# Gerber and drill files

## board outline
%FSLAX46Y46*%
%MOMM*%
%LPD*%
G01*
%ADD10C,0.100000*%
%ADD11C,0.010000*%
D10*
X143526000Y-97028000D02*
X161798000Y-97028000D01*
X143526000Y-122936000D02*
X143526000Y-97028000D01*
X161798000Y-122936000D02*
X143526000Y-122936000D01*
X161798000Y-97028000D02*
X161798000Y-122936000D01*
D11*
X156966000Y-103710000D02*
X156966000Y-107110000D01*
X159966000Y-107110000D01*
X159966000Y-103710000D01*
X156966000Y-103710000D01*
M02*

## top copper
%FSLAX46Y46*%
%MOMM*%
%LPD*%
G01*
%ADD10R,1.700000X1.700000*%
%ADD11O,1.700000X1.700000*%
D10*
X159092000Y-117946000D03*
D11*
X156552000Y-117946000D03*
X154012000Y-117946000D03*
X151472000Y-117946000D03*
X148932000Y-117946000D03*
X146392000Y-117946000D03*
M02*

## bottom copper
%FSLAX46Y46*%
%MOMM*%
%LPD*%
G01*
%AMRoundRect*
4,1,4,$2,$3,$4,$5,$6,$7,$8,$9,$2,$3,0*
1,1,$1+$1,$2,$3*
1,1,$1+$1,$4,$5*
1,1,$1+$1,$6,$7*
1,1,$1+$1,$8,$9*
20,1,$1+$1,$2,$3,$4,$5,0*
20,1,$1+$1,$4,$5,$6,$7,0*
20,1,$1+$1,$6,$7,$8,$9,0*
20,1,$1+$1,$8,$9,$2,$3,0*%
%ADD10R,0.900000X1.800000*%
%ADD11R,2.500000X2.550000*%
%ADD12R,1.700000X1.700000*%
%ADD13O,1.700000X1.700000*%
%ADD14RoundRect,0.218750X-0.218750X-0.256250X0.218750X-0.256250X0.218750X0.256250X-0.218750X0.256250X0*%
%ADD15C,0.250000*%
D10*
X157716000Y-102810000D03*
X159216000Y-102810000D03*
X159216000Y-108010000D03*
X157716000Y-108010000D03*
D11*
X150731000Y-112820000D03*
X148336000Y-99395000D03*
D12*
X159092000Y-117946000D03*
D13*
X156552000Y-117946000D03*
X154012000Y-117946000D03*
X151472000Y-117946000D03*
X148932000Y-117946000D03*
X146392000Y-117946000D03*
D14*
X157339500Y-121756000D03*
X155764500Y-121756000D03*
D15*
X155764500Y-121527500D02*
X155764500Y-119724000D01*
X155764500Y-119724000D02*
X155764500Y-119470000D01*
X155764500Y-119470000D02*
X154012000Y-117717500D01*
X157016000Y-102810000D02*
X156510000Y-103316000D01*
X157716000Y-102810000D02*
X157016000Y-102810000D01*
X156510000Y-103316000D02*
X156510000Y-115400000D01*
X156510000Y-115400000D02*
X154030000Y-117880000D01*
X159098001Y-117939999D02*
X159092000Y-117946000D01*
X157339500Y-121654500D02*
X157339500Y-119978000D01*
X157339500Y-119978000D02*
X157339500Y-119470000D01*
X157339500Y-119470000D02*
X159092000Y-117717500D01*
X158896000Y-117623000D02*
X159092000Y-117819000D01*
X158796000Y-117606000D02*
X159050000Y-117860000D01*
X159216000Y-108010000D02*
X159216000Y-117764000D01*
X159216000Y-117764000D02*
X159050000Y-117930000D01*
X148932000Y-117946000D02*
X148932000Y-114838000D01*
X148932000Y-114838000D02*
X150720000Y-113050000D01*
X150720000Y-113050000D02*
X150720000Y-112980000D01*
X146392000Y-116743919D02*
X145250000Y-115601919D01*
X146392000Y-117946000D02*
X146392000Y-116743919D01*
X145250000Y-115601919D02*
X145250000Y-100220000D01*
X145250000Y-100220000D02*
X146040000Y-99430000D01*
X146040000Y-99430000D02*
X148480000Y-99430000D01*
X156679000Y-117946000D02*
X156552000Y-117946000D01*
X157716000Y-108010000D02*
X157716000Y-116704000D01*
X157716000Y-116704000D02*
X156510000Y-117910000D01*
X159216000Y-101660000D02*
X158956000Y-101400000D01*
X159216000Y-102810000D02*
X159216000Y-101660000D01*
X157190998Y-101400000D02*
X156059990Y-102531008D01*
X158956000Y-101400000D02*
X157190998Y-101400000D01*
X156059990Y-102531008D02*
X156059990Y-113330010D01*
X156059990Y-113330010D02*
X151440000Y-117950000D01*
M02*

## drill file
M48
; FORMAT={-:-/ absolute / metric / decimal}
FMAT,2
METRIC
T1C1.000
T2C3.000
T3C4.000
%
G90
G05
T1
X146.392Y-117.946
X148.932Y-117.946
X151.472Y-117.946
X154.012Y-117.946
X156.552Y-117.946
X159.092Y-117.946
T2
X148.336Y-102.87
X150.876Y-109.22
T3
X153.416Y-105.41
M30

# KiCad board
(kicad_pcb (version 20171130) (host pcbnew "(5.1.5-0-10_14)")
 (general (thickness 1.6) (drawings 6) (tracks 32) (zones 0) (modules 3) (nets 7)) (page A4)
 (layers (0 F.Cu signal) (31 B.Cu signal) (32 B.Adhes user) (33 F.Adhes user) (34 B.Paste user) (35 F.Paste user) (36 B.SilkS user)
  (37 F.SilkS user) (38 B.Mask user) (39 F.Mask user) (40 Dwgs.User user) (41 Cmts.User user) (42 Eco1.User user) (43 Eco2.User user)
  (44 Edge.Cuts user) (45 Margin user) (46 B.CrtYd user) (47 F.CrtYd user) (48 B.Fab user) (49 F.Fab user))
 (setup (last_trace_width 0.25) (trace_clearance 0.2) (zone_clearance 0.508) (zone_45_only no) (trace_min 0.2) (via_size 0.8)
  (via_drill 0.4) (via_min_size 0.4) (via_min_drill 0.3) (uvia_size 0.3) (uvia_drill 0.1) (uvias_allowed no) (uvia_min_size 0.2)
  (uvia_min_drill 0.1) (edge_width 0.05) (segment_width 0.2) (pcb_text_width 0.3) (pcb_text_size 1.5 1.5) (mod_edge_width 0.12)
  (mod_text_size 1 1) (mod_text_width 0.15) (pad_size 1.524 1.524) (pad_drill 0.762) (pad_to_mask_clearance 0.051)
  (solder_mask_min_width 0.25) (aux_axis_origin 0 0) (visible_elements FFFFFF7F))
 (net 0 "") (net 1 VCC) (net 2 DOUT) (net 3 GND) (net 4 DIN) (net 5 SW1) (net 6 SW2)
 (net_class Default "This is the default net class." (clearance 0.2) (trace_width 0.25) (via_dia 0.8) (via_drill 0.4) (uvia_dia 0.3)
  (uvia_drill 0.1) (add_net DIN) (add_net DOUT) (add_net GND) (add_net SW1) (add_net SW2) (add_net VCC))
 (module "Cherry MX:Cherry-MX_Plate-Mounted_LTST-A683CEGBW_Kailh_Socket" (layer F.Cu) (at 153.416 105.41 90)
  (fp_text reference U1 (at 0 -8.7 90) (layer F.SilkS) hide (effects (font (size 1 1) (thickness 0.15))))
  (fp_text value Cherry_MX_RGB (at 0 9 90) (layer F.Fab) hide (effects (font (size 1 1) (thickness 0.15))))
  (fp_poly (pts (xy 1.7 3.55) (xy -1.7 3.55) (xy -1.7 6.55) (xy 1.7 6.55)) (layer Edge.Cuts) (width 0.01))
  (pad 4 smd rect (at 2.6 4.3 90) (size 1.8 0.9) (layers B.Cu B.Paste B.Mask) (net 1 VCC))
  (pad 3 smd rect (at 2.6 5.8 90) (size 1.8 0.9) (layers B.Cu B.Paste B.Mask) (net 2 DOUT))
  (pad 1 smd rect (at -2.6 5.8 90) (size 1.8 0.9) (layers B.Cu B.Paste B.Mask) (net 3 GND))
  (pad 2 smd rect (at -2.6 4.3 90) (size 1.8 0.9) (layers B.Cu B.Paste B.Mask) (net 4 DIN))
  (pad "" np_thru_hole circle (at -3.81 -2.54 90) (size 3 3) (drill 3) (layers *.Cu *.Mask))
  (pad "" np_thru_hole circle (at 2.54 -5.08 90) (size 3 3) (drill 3) (layers *.Cu *.Mask))
  (pad 5 smd rect (at -7.41 -2.685 90) (size 2.55 2.5) (layers B.Cu B.Paste B.Mask) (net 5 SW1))
  (pad 6 smd rect (at 6.015 -5.08 90) (size 2.55 2.5) (layers B.Cu B.Paste B.Mask) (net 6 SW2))
  (pad "" np_thru_hole circle (at 0 0 90) (size 4 4) (drill 4) (layers *.Cu *.Mask)))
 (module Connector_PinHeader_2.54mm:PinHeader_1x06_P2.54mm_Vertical (layer F.Cu) (at 159.092 117.946 270)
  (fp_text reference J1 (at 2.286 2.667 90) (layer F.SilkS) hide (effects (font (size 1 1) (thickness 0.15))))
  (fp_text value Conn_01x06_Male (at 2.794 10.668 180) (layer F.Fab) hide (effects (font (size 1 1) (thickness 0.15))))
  (pad 1 thru_hole rect (at 0 0 270) (size 1.7 1.7) (drill 1) (layers *.Cu *.Mask) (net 3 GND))
  (pad 2 thru_hole oval (at 0 2.54 270) (size 1.7 1.7) (drill 1) (layers *.Cu *.Mask) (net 4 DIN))
  (pad 3 thru_hole oval (at 0 5.08 270) (size 1.7 1.7) (drill 1) (layers *.Cu *.Mask) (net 1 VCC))
  (pad 4 thru_hole oval (at 0 7.62 270) (size 1.7 1.7) (drill 1) (layers *.Cu *.Mask) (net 2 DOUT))
  (pad 5 thru_hole oval (at 0 10.16 270) (size 1.7 1.7) (drill 1) (layers *.Cu *.Mask) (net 5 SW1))
  (pad 6 thru_hole oval (at 0 12.7 270) (size 1.7 1.7) (drill 1) (layers *.Cu *.Mask) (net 6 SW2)))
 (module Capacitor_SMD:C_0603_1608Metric (layer B.Cu) (at 156.552 121.756)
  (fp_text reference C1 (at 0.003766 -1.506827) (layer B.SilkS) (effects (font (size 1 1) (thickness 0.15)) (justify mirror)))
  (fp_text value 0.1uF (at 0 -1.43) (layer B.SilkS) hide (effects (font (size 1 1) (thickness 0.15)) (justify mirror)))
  (pad 2 smd roundrect (at 0.7875 0) (size 0.875 0.95) (layers B.Cu B.Paste B.Mask) (roundrect_rratio 0.25) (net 3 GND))
  (pad 1 smd roundrect (at -0.7875 0) (size 0.875 0.95) (layers B.Cu B.Paste B.Mask) (roundrect_rratio 0.25) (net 1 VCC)))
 (gr_line (start 143.526 97.028) (end 161.798 97.028) (layer Edge.Cuts) (width 0.1))
 (gr_line (start 143.526 122.936) (end 143.526 97.028) (layer Edge.Cuts) (width 0.1))
 (gr_line (start 161.798 122.936) (end 143.526 122.936) (layer Edge.Cuts) (width 0.1))
 (gr_line (start 161.798 97.028) (end 161.798 122.936) (layer Edge.Cuts) (width 0.1))
 (segment (start 155.7645 121.5275) (end 155.7645 119.724) (width 0.25) (layer B.Cu) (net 1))
 (segment (start 155.7645 119.724) (end 155.7645 119.47) (width 0.25) (layer B.Cu) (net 1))
 (segment (start 155.7645 119.47) (end 154.012 117.7175) (width 0.25) (layer B.Cu) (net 1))
 (segment (start 157.016 102.81) (end 156.51 103.316) (width 0.25) (layer B.Cu) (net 1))
 (segment (start 157.716 102.81) (end 157.016 102.81) (width 0.25) (layer B.Cu) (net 1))
 (segment (start 156.51 103.316) (end 156.51 115.4) (width 0.25) (layer B.Cu) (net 1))
 (segment (start 156.51 115.4) (end 154.03 117.88) (width 0.25) (layer B.Cu) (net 1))
 (segment (start 159.098001 117.939999) (end 159.092 117.946) (width 0.25) (layer B.Cu) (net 3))
 (segment (start 157.3395 121.6545) (end 157.3395 119.978) (width 0.25) (layer B.Cu) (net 3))
 (segment (start 157.3395 119.978) (end 157.3395 119.47) (width 0.25) (layer B.Cu) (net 3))
 (segment (start 157.3395 119.47) (end 159.092 117.7175) (width 0.25) (layer B.Cu) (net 3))
 (segment (start 158.896 117.623) (end 159.092 117.819) (width 0.25) (layer B.Cu) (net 3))
 (segment (start 158.796 117.606) (end 159.05 117.86) (width 0.25) (layer B.Cu) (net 3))
 (segment (start 159.216 108.01) (end 159.216 117.764) (width 0.25) (layer B.Cu) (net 3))
 (segment (start 159.216 117.764) (end 159.05 117.93) (width 0.25) (layer B.Cu) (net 3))
 (segment (start 148.932 117.946) (end 148.932 114.838) (width 0.25) (layer B.Cu) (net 5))
 (segment (start 148.932 114.838) (end 150.72 113.05) (width 0.25) (layer B.Cu) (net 5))
 (segment (start 150.72 113.05) (end 150.72 112.98) (width 0.25) (layer B.Cu) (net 5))
 (segment (start 146.392 116.743919) (end 145.25 115.601919) (width 0.25) (layer B.Cu) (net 6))
 (segment (start 146.392 117.946) (end 146.392 116.743919) (width 0.25) (layer B.Cu) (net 6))
 (segment (start 145.25 115.601919) (end 145.25 100.22) (width 0.25) (layer B.Cu) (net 6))
 (segment (start 145.25 100.22) (end 146.04 99.43) (width 0.25) (layer B.Cu) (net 6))
 (segment (start 146.04 99.43) (end 148.48 99.43) (width 0.25) (layer B.Cu) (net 6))
 (segment (start 156.679 117.946) (end 156.552 117.946) (width 0.25) (layer B.Cu) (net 4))
 (segment (start 157.716 108.01) (end 157.716 116.704) (width 0.25) (layer B.Cu) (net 4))
 (segment (start 157.716 116.704) (end 156.51 117.91) (width 0.25) (layer B.Cu) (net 4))
 (segment (start 159.216 101.66) (end 158.956 101.4) (width 0.25) (layer B.Cu) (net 2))
 (segment (start 159.216 102.81) (end 159.216 101.66) (width 0.25) (layer B.Cu) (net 2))
 (segment (start 157.190998 101.4) (end 156.05999 102.531008) (width 0.25) (layer B.Cu) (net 2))
 (segment (start 158.956 101.4) (end 157.190998 101.4) (width 0.25) (layer B.Cu) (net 2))
 (segment (start 156.05999 102.531008) (end 156.05999 113.33001) (width 0.25) (layer B.Cu) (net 2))
 (segment (start 156.05999 113.33001) (end 151.44 117.95) (width 0.25) (layer B.Cu) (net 2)))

